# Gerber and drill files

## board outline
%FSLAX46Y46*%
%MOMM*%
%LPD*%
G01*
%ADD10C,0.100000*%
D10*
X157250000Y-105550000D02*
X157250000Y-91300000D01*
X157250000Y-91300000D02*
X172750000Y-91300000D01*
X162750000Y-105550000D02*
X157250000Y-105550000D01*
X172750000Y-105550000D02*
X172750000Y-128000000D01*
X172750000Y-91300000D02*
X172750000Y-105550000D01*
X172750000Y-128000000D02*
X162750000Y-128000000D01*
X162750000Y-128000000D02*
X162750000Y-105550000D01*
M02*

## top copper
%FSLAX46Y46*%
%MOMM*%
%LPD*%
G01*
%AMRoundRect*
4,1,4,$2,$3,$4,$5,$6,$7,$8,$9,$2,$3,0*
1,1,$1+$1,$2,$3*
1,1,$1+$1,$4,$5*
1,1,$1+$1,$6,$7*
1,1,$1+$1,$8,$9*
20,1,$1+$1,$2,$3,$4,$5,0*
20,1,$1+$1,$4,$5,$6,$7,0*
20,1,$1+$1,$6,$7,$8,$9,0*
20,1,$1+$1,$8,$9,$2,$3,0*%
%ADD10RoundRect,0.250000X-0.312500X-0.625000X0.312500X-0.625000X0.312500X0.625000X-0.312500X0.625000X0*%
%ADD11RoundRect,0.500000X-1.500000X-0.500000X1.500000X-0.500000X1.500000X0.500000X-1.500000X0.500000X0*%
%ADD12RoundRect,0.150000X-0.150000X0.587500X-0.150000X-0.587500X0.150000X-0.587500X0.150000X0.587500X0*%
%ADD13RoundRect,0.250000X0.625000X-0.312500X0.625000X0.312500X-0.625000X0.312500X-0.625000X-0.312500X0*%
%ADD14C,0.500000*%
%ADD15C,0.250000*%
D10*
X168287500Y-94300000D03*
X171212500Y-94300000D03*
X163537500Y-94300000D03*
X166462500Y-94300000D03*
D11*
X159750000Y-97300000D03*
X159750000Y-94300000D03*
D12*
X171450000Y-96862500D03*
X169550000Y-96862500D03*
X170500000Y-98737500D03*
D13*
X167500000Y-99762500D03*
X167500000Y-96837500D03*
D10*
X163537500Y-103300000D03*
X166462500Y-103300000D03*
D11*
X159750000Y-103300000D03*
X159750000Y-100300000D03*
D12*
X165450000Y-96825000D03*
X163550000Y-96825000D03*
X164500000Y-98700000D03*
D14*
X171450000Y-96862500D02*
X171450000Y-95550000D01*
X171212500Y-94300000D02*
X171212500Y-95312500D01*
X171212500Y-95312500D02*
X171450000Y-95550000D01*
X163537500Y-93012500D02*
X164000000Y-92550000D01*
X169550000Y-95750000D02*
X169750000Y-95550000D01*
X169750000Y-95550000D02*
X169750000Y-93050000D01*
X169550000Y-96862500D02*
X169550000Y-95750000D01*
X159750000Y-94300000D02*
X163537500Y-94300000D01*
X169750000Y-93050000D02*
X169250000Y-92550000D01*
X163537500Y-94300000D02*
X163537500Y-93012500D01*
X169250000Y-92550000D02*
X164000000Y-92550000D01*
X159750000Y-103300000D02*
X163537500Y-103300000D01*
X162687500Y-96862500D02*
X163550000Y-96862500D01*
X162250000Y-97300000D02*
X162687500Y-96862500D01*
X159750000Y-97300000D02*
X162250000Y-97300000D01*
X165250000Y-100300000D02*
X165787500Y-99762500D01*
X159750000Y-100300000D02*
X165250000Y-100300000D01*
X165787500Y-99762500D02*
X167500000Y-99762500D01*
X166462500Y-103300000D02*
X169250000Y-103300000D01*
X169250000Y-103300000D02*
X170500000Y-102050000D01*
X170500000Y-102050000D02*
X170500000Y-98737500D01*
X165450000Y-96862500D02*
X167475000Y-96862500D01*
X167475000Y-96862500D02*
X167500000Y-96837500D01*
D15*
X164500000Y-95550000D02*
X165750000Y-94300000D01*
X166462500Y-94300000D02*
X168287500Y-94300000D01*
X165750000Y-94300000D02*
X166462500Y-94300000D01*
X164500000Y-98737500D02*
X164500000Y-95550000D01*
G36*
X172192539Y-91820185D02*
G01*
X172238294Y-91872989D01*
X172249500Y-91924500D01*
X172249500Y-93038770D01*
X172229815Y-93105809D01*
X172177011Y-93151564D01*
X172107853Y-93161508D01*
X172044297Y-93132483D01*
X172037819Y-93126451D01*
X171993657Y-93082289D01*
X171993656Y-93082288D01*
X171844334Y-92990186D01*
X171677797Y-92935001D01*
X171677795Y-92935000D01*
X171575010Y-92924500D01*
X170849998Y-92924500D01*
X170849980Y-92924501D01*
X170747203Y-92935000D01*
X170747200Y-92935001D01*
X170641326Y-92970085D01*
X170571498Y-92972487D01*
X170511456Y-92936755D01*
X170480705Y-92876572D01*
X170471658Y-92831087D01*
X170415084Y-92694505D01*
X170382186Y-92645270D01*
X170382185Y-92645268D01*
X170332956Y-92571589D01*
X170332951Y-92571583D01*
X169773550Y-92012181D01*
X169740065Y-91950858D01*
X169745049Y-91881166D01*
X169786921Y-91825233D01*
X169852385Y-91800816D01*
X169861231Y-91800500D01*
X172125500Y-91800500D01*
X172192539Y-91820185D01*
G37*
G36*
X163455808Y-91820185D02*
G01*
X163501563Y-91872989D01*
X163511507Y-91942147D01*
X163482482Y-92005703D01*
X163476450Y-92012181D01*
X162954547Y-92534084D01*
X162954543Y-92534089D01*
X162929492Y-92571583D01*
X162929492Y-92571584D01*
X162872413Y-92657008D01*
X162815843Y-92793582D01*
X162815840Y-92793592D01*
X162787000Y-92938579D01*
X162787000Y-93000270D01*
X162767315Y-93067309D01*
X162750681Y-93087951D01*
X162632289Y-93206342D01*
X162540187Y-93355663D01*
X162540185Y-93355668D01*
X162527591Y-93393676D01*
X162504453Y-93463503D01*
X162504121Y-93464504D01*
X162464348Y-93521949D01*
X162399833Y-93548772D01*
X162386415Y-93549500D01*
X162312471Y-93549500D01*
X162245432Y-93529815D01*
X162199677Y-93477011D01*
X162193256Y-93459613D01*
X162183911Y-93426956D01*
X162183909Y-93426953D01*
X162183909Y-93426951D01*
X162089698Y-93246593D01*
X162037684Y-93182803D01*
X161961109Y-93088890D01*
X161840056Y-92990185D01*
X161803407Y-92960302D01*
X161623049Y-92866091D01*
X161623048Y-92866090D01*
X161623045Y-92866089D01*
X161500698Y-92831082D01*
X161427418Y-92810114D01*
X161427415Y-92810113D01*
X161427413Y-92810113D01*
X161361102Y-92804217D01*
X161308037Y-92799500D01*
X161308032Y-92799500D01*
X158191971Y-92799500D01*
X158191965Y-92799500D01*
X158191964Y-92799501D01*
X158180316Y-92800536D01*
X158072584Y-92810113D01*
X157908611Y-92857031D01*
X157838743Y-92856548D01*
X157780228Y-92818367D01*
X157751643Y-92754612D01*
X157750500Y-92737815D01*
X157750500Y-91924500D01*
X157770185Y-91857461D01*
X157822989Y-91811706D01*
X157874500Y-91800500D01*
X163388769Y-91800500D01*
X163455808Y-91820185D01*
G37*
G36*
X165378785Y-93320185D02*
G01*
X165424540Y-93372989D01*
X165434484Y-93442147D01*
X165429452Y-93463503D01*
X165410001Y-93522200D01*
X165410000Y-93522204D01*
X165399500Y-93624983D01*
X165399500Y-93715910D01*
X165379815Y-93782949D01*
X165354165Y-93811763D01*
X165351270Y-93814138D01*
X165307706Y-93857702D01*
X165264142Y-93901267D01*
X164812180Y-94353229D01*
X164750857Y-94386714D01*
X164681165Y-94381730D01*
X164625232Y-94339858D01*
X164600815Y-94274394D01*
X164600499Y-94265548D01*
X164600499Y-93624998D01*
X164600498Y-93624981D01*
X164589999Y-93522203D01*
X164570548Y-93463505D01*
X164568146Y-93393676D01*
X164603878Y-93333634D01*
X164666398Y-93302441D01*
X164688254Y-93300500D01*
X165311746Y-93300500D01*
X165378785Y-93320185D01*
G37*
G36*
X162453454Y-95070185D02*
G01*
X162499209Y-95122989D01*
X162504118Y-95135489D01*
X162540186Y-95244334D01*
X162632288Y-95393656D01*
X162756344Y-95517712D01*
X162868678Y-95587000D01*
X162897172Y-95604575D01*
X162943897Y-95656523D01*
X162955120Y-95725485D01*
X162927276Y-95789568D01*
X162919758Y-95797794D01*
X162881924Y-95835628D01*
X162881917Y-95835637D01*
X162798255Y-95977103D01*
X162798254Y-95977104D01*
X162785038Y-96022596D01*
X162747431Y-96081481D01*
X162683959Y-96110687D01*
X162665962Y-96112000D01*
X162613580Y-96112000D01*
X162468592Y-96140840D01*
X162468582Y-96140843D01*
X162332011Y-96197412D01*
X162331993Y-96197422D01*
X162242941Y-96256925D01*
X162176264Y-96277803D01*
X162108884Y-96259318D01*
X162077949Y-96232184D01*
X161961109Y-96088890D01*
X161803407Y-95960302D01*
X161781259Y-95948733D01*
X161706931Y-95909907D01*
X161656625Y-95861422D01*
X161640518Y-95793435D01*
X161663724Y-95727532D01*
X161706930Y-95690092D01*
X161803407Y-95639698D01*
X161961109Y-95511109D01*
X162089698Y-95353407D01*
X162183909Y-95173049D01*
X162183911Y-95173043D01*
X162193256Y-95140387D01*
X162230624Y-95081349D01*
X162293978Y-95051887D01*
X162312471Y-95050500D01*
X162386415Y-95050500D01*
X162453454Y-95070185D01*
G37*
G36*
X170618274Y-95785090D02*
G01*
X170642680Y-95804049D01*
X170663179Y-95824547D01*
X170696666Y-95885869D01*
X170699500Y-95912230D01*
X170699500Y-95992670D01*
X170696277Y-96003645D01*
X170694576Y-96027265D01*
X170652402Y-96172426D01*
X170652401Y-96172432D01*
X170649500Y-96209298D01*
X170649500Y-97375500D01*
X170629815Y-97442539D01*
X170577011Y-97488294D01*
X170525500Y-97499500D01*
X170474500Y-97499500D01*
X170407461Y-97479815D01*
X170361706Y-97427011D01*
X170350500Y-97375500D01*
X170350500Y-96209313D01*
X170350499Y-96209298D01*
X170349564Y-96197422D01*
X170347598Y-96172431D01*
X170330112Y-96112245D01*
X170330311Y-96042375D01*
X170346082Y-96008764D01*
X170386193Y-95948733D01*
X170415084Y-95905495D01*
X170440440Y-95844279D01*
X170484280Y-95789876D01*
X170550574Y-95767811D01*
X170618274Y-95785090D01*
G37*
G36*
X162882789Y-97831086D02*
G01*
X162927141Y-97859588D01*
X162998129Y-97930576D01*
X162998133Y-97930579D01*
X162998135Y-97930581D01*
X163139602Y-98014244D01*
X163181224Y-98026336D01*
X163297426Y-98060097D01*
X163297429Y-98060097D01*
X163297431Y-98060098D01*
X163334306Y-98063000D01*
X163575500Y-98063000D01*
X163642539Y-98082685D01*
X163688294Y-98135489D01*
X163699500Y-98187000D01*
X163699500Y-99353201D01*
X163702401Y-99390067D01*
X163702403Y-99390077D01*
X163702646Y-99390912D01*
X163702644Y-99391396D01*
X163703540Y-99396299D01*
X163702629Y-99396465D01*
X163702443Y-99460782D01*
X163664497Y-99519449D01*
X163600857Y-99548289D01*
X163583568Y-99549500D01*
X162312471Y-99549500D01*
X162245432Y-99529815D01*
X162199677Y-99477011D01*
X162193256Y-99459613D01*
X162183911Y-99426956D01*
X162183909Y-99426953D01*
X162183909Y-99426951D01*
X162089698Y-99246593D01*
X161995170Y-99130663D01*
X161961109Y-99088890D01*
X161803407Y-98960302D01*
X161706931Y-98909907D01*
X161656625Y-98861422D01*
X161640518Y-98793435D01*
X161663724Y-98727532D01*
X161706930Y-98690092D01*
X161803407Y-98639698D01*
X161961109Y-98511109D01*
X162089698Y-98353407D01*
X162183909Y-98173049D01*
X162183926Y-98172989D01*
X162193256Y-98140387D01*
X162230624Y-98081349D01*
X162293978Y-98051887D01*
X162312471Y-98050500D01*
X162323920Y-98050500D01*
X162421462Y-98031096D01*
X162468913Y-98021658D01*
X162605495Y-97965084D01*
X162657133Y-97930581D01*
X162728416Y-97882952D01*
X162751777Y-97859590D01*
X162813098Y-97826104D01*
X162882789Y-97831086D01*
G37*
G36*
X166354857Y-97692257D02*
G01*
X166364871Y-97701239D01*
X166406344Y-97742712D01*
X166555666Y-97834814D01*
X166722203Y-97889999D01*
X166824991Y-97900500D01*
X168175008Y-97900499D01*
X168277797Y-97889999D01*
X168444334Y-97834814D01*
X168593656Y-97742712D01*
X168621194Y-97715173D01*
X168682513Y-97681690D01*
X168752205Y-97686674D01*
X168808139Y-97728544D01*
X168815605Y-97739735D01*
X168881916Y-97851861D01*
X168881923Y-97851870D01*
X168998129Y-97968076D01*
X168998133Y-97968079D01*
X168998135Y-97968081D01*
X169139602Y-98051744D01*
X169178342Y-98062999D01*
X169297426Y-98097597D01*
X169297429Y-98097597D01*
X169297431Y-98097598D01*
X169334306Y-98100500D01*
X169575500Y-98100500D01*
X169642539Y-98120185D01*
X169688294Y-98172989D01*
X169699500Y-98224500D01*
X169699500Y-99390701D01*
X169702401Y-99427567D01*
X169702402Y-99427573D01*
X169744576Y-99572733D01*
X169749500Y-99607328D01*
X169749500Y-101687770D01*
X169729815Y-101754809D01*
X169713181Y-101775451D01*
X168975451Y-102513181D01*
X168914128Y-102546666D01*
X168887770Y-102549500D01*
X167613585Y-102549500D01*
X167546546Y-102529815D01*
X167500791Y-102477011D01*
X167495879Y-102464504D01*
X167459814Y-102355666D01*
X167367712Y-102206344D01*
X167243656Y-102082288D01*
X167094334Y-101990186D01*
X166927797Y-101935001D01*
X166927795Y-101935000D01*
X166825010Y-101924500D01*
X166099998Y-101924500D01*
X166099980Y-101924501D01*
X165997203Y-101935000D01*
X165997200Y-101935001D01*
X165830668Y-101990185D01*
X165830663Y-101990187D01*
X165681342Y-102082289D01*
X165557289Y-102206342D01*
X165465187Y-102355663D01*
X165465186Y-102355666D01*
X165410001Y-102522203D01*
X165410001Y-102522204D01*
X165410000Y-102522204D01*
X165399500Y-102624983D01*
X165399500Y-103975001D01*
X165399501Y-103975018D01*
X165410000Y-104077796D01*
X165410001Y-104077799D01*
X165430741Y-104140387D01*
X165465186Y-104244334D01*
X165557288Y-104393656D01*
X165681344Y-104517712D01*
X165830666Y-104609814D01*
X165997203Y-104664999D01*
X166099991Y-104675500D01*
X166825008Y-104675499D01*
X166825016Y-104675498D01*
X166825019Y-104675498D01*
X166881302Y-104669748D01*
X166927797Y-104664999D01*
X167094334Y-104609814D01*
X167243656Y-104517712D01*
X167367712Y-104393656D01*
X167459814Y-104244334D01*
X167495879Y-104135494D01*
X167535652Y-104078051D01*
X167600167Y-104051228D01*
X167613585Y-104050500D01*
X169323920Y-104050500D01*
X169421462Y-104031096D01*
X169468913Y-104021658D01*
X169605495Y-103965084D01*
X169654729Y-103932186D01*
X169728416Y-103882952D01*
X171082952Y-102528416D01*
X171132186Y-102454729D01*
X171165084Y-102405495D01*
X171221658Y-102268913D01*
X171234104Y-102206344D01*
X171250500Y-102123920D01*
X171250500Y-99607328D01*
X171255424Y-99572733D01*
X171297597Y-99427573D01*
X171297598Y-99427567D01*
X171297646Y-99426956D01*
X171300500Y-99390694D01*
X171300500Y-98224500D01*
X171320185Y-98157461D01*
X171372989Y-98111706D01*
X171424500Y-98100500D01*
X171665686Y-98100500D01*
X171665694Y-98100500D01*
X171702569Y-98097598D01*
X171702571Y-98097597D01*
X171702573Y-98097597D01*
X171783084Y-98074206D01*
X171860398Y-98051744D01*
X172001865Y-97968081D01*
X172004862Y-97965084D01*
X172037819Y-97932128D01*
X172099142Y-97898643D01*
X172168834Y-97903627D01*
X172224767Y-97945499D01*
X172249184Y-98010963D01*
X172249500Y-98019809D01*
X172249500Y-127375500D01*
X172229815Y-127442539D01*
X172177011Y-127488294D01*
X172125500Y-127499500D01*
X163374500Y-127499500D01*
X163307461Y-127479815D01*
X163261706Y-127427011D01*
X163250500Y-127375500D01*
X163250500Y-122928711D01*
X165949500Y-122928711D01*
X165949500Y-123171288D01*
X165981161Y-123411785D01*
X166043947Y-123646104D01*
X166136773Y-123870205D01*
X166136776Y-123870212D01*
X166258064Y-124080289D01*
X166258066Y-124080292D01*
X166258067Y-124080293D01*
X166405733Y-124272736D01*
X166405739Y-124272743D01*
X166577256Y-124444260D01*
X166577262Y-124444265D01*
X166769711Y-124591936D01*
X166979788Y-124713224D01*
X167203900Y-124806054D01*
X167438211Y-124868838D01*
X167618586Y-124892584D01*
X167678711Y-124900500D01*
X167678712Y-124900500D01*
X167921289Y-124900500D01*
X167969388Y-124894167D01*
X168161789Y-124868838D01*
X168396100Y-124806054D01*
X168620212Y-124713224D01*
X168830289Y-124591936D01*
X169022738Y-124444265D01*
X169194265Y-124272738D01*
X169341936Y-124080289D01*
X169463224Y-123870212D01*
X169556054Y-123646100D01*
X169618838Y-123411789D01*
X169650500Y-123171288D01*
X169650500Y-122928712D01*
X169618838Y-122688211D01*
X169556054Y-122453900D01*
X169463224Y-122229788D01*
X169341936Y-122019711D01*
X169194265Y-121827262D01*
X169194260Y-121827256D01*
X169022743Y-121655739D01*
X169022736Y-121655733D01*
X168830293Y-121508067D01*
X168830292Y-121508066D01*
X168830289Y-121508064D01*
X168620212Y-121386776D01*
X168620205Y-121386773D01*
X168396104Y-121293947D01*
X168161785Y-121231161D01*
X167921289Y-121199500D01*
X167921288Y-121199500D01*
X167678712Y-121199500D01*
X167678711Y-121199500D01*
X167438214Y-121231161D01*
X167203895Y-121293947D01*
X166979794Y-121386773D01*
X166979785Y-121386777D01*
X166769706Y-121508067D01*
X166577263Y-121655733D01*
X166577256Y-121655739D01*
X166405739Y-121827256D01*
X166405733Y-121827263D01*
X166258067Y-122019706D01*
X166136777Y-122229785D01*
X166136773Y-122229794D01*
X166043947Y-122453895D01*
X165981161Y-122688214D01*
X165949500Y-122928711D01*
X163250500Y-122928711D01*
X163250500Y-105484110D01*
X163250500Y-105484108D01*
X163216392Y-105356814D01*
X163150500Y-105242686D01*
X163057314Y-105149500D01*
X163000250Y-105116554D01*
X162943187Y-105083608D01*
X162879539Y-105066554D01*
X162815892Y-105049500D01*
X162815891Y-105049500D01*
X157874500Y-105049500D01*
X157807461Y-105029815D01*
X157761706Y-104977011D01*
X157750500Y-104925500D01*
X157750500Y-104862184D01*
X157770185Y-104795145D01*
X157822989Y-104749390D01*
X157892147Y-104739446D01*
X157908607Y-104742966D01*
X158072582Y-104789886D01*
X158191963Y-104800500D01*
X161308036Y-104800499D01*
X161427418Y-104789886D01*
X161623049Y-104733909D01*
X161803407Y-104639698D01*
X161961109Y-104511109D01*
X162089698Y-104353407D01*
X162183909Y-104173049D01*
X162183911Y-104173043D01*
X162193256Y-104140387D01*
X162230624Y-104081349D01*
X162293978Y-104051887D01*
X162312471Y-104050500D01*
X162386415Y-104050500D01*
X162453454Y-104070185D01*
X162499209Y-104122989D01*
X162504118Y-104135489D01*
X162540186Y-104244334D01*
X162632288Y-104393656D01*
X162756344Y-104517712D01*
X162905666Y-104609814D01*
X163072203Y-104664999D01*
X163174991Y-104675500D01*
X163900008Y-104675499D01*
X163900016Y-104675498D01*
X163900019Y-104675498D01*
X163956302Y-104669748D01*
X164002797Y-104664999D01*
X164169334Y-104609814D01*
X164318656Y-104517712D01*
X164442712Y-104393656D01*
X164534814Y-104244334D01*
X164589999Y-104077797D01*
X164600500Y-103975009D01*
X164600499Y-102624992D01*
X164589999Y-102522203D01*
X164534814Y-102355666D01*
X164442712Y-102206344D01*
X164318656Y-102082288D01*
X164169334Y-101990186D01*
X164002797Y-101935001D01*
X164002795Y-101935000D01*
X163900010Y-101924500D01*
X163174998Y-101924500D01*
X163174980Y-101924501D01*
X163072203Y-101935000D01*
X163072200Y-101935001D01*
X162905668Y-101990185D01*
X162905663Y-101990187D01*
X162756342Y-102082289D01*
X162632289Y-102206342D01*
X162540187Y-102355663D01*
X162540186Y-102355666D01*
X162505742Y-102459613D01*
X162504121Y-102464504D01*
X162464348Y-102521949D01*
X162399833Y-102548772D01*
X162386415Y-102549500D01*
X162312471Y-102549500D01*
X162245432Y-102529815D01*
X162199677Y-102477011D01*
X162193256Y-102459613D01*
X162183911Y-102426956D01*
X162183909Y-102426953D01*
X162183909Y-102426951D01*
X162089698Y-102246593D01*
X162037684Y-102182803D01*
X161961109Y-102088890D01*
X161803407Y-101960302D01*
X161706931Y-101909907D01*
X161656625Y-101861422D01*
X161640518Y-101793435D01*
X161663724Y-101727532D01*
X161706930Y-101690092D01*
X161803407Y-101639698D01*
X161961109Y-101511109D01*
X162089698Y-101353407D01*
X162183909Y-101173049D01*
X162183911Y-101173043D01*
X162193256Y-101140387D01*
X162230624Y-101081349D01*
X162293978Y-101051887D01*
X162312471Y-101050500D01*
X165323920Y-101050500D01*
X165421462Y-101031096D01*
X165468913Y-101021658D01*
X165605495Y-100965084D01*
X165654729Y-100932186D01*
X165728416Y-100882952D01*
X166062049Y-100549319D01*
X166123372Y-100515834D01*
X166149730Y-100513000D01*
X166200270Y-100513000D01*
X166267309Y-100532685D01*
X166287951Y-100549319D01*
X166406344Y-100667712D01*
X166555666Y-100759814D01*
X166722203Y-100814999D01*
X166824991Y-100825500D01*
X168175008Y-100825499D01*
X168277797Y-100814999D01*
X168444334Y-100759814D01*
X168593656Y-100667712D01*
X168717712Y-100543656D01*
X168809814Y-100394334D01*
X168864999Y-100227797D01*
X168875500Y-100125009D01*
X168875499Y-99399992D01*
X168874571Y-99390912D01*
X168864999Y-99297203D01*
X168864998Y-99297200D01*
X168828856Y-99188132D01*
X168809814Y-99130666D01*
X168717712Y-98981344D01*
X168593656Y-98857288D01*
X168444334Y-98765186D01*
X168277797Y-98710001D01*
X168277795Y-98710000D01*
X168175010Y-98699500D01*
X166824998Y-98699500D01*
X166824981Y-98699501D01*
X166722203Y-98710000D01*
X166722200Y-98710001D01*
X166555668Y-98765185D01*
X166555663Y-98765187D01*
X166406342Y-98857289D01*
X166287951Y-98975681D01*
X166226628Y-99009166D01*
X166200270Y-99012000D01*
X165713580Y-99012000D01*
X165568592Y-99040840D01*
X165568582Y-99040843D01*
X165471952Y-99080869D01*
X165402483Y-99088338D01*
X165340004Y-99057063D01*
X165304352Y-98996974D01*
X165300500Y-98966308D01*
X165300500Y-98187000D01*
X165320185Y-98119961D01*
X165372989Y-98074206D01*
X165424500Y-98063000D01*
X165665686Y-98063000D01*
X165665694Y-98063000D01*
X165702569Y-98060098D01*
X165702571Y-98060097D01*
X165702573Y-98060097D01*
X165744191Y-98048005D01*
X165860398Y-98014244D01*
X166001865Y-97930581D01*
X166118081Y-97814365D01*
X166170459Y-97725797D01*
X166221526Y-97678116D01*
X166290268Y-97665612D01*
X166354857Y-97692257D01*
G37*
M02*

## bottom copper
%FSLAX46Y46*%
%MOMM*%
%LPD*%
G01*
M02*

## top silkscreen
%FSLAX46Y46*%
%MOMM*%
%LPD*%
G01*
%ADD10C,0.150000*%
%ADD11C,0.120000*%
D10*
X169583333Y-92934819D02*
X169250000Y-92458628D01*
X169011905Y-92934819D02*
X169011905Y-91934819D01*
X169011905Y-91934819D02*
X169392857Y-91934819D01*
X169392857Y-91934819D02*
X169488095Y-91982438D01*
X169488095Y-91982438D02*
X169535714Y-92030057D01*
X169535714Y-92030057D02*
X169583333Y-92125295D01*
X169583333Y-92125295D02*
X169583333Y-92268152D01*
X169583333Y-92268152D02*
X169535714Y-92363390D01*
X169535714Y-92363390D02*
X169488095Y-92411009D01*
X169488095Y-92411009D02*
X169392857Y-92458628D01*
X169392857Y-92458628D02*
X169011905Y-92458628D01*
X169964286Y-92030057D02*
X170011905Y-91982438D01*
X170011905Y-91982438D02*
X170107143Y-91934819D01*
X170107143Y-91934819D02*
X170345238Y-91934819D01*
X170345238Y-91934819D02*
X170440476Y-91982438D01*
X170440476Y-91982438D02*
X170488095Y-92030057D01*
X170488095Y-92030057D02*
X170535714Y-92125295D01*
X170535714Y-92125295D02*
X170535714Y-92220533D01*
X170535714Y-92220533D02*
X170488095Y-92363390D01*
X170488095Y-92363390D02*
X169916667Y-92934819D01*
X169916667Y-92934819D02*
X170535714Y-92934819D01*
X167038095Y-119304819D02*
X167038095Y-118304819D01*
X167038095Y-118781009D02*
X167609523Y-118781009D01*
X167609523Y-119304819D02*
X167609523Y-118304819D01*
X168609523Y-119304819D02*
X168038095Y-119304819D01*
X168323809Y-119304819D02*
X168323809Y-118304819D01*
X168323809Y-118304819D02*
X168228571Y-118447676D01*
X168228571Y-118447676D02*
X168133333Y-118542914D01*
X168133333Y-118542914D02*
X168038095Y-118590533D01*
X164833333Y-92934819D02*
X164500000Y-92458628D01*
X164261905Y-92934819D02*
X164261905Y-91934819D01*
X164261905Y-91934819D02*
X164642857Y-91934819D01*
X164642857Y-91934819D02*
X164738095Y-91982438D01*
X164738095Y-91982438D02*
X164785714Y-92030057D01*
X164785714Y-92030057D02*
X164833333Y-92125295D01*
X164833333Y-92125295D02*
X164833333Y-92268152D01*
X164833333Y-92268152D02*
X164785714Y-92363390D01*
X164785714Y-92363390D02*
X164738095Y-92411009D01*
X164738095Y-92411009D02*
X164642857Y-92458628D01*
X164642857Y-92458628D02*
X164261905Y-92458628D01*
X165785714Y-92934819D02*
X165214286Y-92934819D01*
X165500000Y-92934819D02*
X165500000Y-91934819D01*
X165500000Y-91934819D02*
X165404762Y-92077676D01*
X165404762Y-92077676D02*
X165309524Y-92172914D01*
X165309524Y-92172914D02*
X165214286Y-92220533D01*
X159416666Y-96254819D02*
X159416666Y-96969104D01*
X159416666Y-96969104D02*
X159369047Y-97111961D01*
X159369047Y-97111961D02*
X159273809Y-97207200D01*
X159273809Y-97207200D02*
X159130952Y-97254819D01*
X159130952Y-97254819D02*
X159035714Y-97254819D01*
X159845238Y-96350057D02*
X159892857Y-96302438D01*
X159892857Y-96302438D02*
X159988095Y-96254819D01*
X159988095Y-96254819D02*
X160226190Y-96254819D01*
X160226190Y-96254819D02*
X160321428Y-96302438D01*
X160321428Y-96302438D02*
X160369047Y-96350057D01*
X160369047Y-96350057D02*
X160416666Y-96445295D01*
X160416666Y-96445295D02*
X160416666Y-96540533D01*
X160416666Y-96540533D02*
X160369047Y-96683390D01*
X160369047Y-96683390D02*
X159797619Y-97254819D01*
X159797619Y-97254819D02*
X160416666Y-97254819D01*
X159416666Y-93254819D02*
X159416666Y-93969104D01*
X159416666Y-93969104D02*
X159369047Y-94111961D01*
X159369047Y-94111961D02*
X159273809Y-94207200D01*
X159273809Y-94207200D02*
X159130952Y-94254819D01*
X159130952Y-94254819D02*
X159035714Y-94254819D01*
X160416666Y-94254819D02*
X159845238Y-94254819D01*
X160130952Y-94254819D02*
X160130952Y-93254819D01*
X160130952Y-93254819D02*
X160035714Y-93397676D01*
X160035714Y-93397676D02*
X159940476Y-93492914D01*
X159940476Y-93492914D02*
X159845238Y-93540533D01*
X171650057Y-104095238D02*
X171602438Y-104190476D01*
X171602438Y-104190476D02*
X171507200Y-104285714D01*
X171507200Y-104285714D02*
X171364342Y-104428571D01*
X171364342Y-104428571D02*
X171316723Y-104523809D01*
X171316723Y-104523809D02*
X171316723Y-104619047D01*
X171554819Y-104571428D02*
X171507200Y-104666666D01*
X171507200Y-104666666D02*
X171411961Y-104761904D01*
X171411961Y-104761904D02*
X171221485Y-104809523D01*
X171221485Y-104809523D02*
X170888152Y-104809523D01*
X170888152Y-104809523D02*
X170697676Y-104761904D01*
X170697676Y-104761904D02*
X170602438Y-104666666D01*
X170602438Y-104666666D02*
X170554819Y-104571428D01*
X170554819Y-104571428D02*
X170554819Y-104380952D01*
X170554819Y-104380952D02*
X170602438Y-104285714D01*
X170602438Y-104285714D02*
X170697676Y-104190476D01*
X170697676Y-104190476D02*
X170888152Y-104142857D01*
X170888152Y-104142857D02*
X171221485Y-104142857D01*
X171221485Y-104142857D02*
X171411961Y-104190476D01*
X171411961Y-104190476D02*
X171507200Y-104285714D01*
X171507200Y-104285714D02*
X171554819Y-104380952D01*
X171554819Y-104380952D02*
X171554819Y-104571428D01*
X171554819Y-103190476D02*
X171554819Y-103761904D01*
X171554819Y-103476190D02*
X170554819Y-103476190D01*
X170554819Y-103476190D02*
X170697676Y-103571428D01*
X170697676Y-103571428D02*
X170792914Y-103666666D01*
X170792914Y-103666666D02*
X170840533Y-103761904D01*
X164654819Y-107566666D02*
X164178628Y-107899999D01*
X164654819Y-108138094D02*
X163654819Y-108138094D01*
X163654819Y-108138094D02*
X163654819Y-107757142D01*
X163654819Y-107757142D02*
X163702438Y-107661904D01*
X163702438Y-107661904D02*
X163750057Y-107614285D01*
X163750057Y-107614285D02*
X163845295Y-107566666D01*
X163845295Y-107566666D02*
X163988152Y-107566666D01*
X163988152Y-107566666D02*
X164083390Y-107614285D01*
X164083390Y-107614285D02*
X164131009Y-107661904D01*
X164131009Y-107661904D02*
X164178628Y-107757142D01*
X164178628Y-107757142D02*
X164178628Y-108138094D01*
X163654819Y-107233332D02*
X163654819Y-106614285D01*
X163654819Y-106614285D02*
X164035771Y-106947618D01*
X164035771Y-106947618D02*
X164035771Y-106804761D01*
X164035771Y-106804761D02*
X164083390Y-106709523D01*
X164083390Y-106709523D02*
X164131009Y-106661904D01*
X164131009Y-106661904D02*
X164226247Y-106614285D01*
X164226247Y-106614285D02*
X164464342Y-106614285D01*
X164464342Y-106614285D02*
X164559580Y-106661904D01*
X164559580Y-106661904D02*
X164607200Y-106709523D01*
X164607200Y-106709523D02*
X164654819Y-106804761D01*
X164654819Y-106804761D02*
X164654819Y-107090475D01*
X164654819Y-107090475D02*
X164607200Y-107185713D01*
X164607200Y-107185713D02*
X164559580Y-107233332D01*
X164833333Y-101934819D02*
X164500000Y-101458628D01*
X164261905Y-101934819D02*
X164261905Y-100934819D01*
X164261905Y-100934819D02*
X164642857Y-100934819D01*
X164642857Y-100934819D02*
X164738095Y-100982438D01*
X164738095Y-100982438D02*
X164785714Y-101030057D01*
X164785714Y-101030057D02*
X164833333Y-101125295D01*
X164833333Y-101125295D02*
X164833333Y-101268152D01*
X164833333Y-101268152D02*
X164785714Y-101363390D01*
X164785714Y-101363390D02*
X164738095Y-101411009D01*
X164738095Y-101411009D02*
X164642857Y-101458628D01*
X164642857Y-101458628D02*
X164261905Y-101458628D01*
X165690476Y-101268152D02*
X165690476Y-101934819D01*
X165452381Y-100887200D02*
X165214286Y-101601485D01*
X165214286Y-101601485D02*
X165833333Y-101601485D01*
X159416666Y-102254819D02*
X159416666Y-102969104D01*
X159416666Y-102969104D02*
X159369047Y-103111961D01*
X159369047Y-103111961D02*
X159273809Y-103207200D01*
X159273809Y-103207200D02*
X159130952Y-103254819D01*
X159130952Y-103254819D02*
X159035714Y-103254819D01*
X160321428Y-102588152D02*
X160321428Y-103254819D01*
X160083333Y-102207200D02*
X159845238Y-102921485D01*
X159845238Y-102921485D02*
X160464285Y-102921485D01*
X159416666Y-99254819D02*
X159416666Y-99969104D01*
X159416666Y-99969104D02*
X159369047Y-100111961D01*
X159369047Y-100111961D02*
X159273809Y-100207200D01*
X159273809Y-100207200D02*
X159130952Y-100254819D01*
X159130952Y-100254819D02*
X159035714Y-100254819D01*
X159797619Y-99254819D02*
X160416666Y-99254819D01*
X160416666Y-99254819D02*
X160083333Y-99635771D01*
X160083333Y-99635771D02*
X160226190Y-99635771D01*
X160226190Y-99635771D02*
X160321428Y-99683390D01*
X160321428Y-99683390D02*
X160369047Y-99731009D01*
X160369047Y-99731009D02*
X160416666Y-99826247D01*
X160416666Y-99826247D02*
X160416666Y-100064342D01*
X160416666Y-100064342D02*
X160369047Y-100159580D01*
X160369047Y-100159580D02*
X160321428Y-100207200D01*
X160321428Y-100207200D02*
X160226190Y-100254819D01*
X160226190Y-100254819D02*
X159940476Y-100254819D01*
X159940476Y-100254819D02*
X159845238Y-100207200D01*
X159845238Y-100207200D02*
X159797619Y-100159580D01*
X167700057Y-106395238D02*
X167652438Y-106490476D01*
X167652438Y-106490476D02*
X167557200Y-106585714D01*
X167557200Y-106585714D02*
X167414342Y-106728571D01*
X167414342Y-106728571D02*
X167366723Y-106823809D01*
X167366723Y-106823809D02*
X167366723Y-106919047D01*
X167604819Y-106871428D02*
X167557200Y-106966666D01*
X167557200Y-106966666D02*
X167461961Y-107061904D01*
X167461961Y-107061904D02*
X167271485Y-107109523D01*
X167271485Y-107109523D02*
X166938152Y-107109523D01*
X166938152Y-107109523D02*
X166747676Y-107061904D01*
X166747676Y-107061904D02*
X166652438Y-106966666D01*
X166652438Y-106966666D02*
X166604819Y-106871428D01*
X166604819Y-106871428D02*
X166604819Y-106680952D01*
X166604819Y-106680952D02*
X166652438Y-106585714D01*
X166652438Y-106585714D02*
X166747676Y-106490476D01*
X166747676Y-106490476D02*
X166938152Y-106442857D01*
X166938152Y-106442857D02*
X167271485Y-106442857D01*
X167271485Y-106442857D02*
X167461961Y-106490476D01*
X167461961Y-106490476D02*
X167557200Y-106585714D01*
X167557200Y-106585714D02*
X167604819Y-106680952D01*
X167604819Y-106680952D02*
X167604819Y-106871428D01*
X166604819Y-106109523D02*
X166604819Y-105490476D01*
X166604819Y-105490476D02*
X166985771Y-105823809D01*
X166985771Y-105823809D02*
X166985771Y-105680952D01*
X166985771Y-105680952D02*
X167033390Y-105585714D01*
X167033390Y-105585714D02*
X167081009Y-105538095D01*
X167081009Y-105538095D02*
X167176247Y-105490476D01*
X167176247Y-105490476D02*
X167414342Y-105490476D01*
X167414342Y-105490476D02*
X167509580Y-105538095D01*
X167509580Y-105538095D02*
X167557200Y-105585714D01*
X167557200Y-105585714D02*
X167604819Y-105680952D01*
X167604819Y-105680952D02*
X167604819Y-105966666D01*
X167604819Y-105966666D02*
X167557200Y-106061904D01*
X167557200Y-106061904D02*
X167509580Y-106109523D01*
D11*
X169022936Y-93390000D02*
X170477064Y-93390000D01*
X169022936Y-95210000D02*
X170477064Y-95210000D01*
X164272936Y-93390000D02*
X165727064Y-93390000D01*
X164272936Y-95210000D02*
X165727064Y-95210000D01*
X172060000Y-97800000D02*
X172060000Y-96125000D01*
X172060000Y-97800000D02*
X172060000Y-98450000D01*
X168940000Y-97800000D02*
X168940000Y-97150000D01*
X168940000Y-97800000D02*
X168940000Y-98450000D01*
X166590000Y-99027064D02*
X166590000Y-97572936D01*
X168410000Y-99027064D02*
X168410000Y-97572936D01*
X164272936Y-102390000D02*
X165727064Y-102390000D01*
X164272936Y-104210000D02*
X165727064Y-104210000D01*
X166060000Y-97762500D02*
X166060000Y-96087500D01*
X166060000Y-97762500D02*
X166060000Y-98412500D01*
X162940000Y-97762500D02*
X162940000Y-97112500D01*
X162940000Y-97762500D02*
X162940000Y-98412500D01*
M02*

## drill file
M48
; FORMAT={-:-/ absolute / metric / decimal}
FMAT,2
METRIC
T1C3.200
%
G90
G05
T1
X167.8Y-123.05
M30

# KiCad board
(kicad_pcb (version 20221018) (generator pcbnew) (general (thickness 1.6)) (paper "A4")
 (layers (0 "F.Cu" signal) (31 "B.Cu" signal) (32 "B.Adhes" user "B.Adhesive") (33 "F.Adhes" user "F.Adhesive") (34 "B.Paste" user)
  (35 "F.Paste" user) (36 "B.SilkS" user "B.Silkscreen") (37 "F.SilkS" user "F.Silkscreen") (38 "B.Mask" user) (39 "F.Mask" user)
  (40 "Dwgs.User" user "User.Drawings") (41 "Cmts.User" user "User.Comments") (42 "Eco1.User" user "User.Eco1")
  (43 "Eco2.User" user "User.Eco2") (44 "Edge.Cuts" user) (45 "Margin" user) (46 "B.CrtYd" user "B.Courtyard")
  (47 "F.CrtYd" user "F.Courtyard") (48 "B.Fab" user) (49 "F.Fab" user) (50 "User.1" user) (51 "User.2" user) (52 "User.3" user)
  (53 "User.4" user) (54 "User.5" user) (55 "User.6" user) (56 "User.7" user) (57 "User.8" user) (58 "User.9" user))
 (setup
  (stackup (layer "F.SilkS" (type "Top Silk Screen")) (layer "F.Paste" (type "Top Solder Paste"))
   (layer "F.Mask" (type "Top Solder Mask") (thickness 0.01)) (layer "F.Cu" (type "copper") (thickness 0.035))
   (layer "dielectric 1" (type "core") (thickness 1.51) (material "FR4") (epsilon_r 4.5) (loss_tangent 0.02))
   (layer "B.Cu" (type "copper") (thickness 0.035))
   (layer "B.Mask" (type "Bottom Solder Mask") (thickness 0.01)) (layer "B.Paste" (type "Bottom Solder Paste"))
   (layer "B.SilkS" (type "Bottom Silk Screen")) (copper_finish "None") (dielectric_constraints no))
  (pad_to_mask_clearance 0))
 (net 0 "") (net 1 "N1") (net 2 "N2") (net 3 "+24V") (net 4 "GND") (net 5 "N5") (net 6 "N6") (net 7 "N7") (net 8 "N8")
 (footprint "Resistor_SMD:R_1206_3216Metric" (layer "F.Cu") (at 169.75 94.3)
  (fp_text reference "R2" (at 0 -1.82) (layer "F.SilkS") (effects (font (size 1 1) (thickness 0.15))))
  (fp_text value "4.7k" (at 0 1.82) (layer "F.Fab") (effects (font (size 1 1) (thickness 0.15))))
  (fp_line (start -0.727064 -0.91) (end 0.727064 -0.91) (stroke (width 0.12) (type solid)) (layer "F.SilkS"))
  (fp_line (start -0.727064 0.91) (end 0.727064 0.91) (stroke (width 0.12) (type solid)) (layer "F.SilkS"))
  (pad "1" smd roundrect (at -1.4625 0) (size 1.125 1.75) (layers "F.Cu" "F.Paste" "F.Mask") (roundrect_rratio 0.222222) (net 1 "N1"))
  (pad "2" smd roundrect (at 1.4625 0) (size 1.125 1.75) (layers "F.Cu" "F.Paste" "F.Mask") (roundrect_rratio 0.222222) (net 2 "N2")))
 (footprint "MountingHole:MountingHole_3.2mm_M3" (layer "F.Cu") (at 167.8 123.05)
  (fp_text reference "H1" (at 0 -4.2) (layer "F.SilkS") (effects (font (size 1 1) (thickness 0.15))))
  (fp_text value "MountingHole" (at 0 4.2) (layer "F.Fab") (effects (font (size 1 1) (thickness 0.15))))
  (pad "" np_thru_hole circle (at 0 0) (size 3.2 3.2) (drill 3.2) (layers "*.Cu" "*.Mask")))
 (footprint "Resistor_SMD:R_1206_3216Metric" (layer "F.Cu") (at 165 94.3)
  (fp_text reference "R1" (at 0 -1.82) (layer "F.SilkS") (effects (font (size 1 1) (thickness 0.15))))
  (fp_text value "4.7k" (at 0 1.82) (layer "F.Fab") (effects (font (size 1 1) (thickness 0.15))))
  (fp_line (start -0.727064 -0.91) (end 0.727064 -0.91) (stroke (width 0.12) (type solid)) (layer "F.SilkS"))
  (fp_line (start -0.727064 0.91) (end 0.727064 0.91) (stroke (width 0.12) (type solid)) (layer "F.SilkS"))
  (pad "1" smd roundrect (at -1.4625 0) (size 1.125 1.75) (layers "F.Cu" "F.Paste" "F.Mask") (roundrect_rratio 0.222222) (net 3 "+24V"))
  (pad "2" smd roundrect (at 1.4625 0) (size 1.125 1.75) (layers "F.Cu" "F.Paste" "F.Mask") (roundrect_rratio 0.222222) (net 1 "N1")))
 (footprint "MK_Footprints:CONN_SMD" (layer "F.Cu") (at 159.75 97.3)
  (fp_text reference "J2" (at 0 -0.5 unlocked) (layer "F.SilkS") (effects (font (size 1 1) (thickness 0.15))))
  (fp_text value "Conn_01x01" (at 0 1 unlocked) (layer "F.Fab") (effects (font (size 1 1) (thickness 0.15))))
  (pad "1" smd roundrect (at 0 0) (size 4 2) (layers "F.Cu" "F.Paste" "F.Mask") (roundrect_rratio 0.25) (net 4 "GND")
   (thermal_bridge_angle 45)))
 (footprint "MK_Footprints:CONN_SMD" (layer "F.Cu") (at 159.75 94.3)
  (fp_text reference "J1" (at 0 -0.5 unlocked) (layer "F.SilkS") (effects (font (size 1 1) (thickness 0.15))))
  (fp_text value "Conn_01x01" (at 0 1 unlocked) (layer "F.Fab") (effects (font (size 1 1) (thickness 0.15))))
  (pad "1" smd roundrect (at 0 0) (size 4 2) (layers "F.Cu" "F.Paste" "F.Mask") (roundrect_rratio 0.25) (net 3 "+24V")
   (thermal_bridge_angle 45)))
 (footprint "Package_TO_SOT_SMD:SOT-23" (layer "F.Cu") (at 170.5 97.8 -90)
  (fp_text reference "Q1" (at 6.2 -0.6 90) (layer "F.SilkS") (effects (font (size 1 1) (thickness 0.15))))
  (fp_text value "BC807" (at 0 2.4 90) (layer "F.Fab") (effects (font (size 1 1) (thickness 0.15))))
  (fp_line (start 0 -1.56) (end -1.675 -1.56) (stroke (width 0.12) (type solid)) (layer "F.SilkS"))
  (fp_line (start 0 -1.56) (end 0.65 -1.56) (stroke (width 0.12) (type solid)) (layer "F.SilkS"))
  (fp_line (start 0 1.56) (end -0.65 1.56) (stroke (width 0.12) (type solid)) (layer "F.SilkS"))
  (fp_line (start 0 1.56) (end 0.65 1.56) (stroke (width 0.12) (type solid)) (layer "F.SilkS"))
  (pad "1" smd roundrect (at -0.9375 -0.95 270) (size 1.475 0.6) (layers "F.Cu" "F.Paste" "F.Mask") (roundrect_rratio 0.25) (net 2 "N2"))
  (pad "2" smd roundrect (at -0.9375 0.95 270) (size 1.475 0.6) (layers "F.Cu" "F.Paste" "F.Mask") (roundrect_rratio 0.25) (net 3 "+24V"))
  (pad "3" smd roundrect (at 0.9375 0 270) (size 1.475 0.6) (layers "F.Cu" "F.Paste" "F.Mask") (roundrect_rratio 0.25) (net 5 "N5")))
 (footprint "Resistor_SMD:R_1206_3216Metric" (layer "F.Cu") (at 167.5 98.3 90)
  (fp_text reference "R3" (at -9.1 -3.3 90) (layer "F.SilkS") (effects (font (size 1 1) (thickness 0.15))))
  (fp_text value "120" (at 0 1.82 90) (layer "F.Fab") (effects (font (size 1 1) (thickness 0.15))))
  (fp_line (start -0.727064 -0.91) (end 0.727064 -0.91) (stroke (width 0.12) (type solid)) (layer "F.SilkS"))
  (fp_line (start -0.727064 0.91) (end 0.727064 0.91) (stroke (width 0.12) (type solid)) (layer "F.SilkS"))
  (pad "1" smd roundrect (at -1.4625 0 90) (size 1.125 1.75) (layers "F.Cu" "F.Paste" "F.Mask") (roundrect_rratio 0.222222) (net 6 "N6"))
  (pad "2" smd roundrect (at 1.4625 0 90) (size 1.125 1.75) (layers "F.Cu" "F.Paste" "F.Mask") (roundrect_rratio 0.222222) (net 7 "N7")))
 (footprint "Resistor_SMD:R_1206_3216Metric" (layer "F.Cu") (at 165 103.3)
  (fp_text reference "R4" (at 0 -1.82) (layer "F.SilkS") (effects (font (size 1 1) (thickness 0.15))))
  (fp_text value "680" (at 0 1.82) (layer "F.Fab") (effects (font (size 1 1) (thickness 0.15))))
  (fp_line (start -0.727064 -0.91) (end 0.727064 -0.91) (stroke (width 0.12) (type solid)) (layer "F.SilkS"))
  (fp_line (start -0.727064 0.91) (end 0.727064 0.91) (stroke (width 0.12) (type solid)) (layer "F.SilkS"))
  (pad "1" smd roundrect (at -1.4625 0) (size 1.125 1.75) (layers "F.Cu" "F.Paste" "F.Mask") (roundrect_rratio 0.222222) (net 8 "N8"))
  (pad "2" smd roundrect (at 1.4625 0) (size 1.125 1.75) (layers "F.Cu" "F.Paste" "F.Mask") (roundrect_rratio 0.222222) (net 5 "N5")))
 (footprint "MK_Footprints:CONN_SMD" (layer "F.Cu") (at 159.75 103.3)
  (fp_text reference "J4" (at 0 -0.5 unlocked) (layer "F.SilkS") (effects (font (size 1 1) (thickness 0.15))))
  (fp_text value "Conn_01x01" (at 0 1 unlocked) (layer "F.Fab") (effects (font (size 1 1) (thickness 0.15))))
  (pad "1" smd roundrect (at 0 0) (size 4 2) (layers "F.Cu" "F.Paste" "F.Mask") (roundrect_rratio 0.25) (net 8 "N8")
   (thermal_bridge_angle 45)))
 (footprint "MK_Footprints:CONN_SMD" (layer "F.Cu") (at 159.75 100.3)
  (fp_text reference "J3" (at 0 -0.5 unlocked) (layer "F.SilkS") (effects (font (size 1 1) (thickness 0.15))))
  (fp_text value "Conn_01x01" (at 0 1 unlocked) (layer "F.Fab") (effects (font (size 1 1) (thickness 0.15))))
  (pad "1" smd roundrect (at 0 0) (size 4 2) (layers "F.Cu" "F.Paste" "F.Mask") (roundrect_rratio 0.25) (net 6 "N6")
   (thermal_bridge_angle 45)))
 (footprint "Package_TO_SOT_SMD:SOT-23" (layer "F.Cu") (at 164.5 97.7625 -90)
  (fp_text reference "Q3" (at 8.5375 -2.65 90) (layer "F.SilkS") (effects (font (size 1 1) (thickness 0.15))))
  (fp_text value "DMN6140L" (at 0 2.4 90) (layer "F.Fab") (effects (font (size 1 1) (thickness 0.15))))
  (fp_line (start 0 -1.56) (end -1.675 -1.56) (stroke (width 0.12) (type solid)) (layer "F.SilkS"))
  (fp_line (start 0 -1.56) (end 0.65 -1.56) (stroke (width 0.12) (type solid)) (layer "F.SilkS"))
  (fp_line (start 0 1.56) (end -0.65 1.56) (stroke (width 0.12) (type solid)) (layer "F.SilkS"))
  (fp_line (start 0 1.56) (end 0.65 1.56) (stroke (width 0.12) (type solid)) (layer "F.SilkS"))
  (pad "1" smd roundrect (at -0.9375 -0.95 270) (size 1.475 0.6) (layers "F.Cu" "F.Paste" "F.Mask") (roundrect_rratio 0.25) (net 7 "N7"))
  (pad "2" smd roundrect (at -0.9375 0.95 270) (size 1.475 0.6) (layers "F.Cu" "F.Paste" "F.Mask") (roundrect_rratio 0.25) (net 4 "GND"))
  (pad "3" smd roundrect (at 0.9375 0 270) (size 1.475 0.6) (layers "F.Cu" "F.Paste" "F.Mask") (roundrect_rratio 0.25) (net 1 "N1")))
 (gr_line (start 157.25 105.55) (end 157.25 91.3) (stroke (width 0.1) (type default)) (layer "Edge.Cuts"))
 (gr_line (start 157.25 91.3) (end 172.75 91.3) (stroke (width 0.1) (type default)) (layer "Edge.Cuts"))
 (gr_line (start 162.75 105.55) (end 157.25 105.55) (stroke (width 0.1) (type default)) (layer "Edge.Cuts"))
 (gr_line (start 172.75 105.55) (end 172.75 128) (stroke (width 0.1) (type default)) (layer "Edge.Cuts"))
 (gr_line (start 172.75 91.3) (end 172.75 105.55) (stroke (width 0.1) (type default)) (layer "Edge.Cuts"))
 (gr_line (start 172.75 128) (end 162.75 128) (stroke (width 0.1) (type default)) (layer "Edge.Cuts"))
 (gr_line (start 162.75 128) (end 162.75 105.55) (stroke (width 0.1) (type default)) (layer "Edge.Cuts"))
 (segment (start 171.45 96.8625) (end 171.45 95.55) (width 0.5) (layer "F.Cu") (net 2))
 (segment (start 171.2125 94.3) (end 171.2125 95.3125) (width 0.5) (layer "F.Cu") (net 2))
 (segment (start 171.2125 95.3125) (end 171.45 95.55) (width 0.5) (layer "F.Cu") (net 2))
 (segment (start 163.5375 93.0125) (end 164 92.55) (width 0.5) (layer "F.Cu") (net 3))
 (segment (start 169.55 95.75) (end 169.75 95.55) (width 0.5) (layer "F.Cu") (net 3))
 (segment (start 169.75 95.55) (end 169.75 93.05) (width 0.5) (layer "F.Cu") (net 3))
 (segment (start 169.55 96.8625) (end 169.55 95.75) (width 0.5) (layer "F.Cu") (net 3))
 (segment (start 159.75 94.3) (end 163.5375 94.3) (width 0.5) (layer "F.Cu") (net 3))
 (segment (start 169.75 93.05) (end 169.25 92.55) (width 0.5) (layer "F.Cu") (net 3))
 (segment (start 163.5375 94.3) (end 163.5375 93.0125) (width 0.5) (layer "F.Cu") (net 3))
 (segment (start 169.25 92.55) (end 164 92.55) (width 0.5) (layer "F.Cu") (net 3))
 (segment (start 159.75 103.3) (end 163.5375 103.3) (width 0.5) (layer "F.Cu") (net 8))
 (segment (start 162.6875 96.8625) (end 163.55 96.8625) (width 0.5) (layer "F.Cu") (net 4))
 (segment (start 162.25 97.3) (end 162.6875 96.8625) (width 0.5) (layer "F.Cu") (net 4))
 (segment (start 159.75 97.3) (end 162.25 97.3) (width 0.5) (layer "F.Cu") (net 4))
 (segment (start 165.25 100.3) (end 165.7875 99.7625) (width 0.5) (layer "F.Cu") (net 6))
 (segment (start 159.75 100.3) (end 165.25 100.3) (width 0.5) (layer "F.Cu") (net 6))
 (segment (start 165.7875 99.7625) (end 167.5 99.7625) (width 0.5) (layer "F.Cu") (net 6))
 (segment (start 166.4625 103.3) (end 169.25 103.3) (width 0.5) (layer "F.Cu") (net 5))
 (segment (start 169.25 103.3) (end 170.5 102.05) (width 0.5) (layer "F.Cu") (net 5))
 (segment (start 170.5 102.05) (end 170.5 98.7375) (width 0.5) (layer "F.Cu") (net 5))
 (segment (start 165.45 96.8625) (end 167.475 96.8625) (width 0.5) (layer "F.Cu") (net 7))
 (segment (start 167.475 96.8625) (end 167.5 96.8375) (width 0.5) (layer "F.Cu") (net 7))
 (segment (start 164.5 95.55) (end 165.75 94.3) (width 0.25) (layer "F.Cu") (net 1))
 (segment (start 166.4625 94.3) (end 168.2875 94.3) (width 0.25) (layer "F.Cu") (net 1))
 (segment (start 165.75 94.3) (end 166.4625 94.3) (width 0.25) (layer "F.Cu") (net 1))
 (segment (start 164.5 98.7375) (end 164.5 95.55) (width 0.25) (layer "F.Cu") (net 1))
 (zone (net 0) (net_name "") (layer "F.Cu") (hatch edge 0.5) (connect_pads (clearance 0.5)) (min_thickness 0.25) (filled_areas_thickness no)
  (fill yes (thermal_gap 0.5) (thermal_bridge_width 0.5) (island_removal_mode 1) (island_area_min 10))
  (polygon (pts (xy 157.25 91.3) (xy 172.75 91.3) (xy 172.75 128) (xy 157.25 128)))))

